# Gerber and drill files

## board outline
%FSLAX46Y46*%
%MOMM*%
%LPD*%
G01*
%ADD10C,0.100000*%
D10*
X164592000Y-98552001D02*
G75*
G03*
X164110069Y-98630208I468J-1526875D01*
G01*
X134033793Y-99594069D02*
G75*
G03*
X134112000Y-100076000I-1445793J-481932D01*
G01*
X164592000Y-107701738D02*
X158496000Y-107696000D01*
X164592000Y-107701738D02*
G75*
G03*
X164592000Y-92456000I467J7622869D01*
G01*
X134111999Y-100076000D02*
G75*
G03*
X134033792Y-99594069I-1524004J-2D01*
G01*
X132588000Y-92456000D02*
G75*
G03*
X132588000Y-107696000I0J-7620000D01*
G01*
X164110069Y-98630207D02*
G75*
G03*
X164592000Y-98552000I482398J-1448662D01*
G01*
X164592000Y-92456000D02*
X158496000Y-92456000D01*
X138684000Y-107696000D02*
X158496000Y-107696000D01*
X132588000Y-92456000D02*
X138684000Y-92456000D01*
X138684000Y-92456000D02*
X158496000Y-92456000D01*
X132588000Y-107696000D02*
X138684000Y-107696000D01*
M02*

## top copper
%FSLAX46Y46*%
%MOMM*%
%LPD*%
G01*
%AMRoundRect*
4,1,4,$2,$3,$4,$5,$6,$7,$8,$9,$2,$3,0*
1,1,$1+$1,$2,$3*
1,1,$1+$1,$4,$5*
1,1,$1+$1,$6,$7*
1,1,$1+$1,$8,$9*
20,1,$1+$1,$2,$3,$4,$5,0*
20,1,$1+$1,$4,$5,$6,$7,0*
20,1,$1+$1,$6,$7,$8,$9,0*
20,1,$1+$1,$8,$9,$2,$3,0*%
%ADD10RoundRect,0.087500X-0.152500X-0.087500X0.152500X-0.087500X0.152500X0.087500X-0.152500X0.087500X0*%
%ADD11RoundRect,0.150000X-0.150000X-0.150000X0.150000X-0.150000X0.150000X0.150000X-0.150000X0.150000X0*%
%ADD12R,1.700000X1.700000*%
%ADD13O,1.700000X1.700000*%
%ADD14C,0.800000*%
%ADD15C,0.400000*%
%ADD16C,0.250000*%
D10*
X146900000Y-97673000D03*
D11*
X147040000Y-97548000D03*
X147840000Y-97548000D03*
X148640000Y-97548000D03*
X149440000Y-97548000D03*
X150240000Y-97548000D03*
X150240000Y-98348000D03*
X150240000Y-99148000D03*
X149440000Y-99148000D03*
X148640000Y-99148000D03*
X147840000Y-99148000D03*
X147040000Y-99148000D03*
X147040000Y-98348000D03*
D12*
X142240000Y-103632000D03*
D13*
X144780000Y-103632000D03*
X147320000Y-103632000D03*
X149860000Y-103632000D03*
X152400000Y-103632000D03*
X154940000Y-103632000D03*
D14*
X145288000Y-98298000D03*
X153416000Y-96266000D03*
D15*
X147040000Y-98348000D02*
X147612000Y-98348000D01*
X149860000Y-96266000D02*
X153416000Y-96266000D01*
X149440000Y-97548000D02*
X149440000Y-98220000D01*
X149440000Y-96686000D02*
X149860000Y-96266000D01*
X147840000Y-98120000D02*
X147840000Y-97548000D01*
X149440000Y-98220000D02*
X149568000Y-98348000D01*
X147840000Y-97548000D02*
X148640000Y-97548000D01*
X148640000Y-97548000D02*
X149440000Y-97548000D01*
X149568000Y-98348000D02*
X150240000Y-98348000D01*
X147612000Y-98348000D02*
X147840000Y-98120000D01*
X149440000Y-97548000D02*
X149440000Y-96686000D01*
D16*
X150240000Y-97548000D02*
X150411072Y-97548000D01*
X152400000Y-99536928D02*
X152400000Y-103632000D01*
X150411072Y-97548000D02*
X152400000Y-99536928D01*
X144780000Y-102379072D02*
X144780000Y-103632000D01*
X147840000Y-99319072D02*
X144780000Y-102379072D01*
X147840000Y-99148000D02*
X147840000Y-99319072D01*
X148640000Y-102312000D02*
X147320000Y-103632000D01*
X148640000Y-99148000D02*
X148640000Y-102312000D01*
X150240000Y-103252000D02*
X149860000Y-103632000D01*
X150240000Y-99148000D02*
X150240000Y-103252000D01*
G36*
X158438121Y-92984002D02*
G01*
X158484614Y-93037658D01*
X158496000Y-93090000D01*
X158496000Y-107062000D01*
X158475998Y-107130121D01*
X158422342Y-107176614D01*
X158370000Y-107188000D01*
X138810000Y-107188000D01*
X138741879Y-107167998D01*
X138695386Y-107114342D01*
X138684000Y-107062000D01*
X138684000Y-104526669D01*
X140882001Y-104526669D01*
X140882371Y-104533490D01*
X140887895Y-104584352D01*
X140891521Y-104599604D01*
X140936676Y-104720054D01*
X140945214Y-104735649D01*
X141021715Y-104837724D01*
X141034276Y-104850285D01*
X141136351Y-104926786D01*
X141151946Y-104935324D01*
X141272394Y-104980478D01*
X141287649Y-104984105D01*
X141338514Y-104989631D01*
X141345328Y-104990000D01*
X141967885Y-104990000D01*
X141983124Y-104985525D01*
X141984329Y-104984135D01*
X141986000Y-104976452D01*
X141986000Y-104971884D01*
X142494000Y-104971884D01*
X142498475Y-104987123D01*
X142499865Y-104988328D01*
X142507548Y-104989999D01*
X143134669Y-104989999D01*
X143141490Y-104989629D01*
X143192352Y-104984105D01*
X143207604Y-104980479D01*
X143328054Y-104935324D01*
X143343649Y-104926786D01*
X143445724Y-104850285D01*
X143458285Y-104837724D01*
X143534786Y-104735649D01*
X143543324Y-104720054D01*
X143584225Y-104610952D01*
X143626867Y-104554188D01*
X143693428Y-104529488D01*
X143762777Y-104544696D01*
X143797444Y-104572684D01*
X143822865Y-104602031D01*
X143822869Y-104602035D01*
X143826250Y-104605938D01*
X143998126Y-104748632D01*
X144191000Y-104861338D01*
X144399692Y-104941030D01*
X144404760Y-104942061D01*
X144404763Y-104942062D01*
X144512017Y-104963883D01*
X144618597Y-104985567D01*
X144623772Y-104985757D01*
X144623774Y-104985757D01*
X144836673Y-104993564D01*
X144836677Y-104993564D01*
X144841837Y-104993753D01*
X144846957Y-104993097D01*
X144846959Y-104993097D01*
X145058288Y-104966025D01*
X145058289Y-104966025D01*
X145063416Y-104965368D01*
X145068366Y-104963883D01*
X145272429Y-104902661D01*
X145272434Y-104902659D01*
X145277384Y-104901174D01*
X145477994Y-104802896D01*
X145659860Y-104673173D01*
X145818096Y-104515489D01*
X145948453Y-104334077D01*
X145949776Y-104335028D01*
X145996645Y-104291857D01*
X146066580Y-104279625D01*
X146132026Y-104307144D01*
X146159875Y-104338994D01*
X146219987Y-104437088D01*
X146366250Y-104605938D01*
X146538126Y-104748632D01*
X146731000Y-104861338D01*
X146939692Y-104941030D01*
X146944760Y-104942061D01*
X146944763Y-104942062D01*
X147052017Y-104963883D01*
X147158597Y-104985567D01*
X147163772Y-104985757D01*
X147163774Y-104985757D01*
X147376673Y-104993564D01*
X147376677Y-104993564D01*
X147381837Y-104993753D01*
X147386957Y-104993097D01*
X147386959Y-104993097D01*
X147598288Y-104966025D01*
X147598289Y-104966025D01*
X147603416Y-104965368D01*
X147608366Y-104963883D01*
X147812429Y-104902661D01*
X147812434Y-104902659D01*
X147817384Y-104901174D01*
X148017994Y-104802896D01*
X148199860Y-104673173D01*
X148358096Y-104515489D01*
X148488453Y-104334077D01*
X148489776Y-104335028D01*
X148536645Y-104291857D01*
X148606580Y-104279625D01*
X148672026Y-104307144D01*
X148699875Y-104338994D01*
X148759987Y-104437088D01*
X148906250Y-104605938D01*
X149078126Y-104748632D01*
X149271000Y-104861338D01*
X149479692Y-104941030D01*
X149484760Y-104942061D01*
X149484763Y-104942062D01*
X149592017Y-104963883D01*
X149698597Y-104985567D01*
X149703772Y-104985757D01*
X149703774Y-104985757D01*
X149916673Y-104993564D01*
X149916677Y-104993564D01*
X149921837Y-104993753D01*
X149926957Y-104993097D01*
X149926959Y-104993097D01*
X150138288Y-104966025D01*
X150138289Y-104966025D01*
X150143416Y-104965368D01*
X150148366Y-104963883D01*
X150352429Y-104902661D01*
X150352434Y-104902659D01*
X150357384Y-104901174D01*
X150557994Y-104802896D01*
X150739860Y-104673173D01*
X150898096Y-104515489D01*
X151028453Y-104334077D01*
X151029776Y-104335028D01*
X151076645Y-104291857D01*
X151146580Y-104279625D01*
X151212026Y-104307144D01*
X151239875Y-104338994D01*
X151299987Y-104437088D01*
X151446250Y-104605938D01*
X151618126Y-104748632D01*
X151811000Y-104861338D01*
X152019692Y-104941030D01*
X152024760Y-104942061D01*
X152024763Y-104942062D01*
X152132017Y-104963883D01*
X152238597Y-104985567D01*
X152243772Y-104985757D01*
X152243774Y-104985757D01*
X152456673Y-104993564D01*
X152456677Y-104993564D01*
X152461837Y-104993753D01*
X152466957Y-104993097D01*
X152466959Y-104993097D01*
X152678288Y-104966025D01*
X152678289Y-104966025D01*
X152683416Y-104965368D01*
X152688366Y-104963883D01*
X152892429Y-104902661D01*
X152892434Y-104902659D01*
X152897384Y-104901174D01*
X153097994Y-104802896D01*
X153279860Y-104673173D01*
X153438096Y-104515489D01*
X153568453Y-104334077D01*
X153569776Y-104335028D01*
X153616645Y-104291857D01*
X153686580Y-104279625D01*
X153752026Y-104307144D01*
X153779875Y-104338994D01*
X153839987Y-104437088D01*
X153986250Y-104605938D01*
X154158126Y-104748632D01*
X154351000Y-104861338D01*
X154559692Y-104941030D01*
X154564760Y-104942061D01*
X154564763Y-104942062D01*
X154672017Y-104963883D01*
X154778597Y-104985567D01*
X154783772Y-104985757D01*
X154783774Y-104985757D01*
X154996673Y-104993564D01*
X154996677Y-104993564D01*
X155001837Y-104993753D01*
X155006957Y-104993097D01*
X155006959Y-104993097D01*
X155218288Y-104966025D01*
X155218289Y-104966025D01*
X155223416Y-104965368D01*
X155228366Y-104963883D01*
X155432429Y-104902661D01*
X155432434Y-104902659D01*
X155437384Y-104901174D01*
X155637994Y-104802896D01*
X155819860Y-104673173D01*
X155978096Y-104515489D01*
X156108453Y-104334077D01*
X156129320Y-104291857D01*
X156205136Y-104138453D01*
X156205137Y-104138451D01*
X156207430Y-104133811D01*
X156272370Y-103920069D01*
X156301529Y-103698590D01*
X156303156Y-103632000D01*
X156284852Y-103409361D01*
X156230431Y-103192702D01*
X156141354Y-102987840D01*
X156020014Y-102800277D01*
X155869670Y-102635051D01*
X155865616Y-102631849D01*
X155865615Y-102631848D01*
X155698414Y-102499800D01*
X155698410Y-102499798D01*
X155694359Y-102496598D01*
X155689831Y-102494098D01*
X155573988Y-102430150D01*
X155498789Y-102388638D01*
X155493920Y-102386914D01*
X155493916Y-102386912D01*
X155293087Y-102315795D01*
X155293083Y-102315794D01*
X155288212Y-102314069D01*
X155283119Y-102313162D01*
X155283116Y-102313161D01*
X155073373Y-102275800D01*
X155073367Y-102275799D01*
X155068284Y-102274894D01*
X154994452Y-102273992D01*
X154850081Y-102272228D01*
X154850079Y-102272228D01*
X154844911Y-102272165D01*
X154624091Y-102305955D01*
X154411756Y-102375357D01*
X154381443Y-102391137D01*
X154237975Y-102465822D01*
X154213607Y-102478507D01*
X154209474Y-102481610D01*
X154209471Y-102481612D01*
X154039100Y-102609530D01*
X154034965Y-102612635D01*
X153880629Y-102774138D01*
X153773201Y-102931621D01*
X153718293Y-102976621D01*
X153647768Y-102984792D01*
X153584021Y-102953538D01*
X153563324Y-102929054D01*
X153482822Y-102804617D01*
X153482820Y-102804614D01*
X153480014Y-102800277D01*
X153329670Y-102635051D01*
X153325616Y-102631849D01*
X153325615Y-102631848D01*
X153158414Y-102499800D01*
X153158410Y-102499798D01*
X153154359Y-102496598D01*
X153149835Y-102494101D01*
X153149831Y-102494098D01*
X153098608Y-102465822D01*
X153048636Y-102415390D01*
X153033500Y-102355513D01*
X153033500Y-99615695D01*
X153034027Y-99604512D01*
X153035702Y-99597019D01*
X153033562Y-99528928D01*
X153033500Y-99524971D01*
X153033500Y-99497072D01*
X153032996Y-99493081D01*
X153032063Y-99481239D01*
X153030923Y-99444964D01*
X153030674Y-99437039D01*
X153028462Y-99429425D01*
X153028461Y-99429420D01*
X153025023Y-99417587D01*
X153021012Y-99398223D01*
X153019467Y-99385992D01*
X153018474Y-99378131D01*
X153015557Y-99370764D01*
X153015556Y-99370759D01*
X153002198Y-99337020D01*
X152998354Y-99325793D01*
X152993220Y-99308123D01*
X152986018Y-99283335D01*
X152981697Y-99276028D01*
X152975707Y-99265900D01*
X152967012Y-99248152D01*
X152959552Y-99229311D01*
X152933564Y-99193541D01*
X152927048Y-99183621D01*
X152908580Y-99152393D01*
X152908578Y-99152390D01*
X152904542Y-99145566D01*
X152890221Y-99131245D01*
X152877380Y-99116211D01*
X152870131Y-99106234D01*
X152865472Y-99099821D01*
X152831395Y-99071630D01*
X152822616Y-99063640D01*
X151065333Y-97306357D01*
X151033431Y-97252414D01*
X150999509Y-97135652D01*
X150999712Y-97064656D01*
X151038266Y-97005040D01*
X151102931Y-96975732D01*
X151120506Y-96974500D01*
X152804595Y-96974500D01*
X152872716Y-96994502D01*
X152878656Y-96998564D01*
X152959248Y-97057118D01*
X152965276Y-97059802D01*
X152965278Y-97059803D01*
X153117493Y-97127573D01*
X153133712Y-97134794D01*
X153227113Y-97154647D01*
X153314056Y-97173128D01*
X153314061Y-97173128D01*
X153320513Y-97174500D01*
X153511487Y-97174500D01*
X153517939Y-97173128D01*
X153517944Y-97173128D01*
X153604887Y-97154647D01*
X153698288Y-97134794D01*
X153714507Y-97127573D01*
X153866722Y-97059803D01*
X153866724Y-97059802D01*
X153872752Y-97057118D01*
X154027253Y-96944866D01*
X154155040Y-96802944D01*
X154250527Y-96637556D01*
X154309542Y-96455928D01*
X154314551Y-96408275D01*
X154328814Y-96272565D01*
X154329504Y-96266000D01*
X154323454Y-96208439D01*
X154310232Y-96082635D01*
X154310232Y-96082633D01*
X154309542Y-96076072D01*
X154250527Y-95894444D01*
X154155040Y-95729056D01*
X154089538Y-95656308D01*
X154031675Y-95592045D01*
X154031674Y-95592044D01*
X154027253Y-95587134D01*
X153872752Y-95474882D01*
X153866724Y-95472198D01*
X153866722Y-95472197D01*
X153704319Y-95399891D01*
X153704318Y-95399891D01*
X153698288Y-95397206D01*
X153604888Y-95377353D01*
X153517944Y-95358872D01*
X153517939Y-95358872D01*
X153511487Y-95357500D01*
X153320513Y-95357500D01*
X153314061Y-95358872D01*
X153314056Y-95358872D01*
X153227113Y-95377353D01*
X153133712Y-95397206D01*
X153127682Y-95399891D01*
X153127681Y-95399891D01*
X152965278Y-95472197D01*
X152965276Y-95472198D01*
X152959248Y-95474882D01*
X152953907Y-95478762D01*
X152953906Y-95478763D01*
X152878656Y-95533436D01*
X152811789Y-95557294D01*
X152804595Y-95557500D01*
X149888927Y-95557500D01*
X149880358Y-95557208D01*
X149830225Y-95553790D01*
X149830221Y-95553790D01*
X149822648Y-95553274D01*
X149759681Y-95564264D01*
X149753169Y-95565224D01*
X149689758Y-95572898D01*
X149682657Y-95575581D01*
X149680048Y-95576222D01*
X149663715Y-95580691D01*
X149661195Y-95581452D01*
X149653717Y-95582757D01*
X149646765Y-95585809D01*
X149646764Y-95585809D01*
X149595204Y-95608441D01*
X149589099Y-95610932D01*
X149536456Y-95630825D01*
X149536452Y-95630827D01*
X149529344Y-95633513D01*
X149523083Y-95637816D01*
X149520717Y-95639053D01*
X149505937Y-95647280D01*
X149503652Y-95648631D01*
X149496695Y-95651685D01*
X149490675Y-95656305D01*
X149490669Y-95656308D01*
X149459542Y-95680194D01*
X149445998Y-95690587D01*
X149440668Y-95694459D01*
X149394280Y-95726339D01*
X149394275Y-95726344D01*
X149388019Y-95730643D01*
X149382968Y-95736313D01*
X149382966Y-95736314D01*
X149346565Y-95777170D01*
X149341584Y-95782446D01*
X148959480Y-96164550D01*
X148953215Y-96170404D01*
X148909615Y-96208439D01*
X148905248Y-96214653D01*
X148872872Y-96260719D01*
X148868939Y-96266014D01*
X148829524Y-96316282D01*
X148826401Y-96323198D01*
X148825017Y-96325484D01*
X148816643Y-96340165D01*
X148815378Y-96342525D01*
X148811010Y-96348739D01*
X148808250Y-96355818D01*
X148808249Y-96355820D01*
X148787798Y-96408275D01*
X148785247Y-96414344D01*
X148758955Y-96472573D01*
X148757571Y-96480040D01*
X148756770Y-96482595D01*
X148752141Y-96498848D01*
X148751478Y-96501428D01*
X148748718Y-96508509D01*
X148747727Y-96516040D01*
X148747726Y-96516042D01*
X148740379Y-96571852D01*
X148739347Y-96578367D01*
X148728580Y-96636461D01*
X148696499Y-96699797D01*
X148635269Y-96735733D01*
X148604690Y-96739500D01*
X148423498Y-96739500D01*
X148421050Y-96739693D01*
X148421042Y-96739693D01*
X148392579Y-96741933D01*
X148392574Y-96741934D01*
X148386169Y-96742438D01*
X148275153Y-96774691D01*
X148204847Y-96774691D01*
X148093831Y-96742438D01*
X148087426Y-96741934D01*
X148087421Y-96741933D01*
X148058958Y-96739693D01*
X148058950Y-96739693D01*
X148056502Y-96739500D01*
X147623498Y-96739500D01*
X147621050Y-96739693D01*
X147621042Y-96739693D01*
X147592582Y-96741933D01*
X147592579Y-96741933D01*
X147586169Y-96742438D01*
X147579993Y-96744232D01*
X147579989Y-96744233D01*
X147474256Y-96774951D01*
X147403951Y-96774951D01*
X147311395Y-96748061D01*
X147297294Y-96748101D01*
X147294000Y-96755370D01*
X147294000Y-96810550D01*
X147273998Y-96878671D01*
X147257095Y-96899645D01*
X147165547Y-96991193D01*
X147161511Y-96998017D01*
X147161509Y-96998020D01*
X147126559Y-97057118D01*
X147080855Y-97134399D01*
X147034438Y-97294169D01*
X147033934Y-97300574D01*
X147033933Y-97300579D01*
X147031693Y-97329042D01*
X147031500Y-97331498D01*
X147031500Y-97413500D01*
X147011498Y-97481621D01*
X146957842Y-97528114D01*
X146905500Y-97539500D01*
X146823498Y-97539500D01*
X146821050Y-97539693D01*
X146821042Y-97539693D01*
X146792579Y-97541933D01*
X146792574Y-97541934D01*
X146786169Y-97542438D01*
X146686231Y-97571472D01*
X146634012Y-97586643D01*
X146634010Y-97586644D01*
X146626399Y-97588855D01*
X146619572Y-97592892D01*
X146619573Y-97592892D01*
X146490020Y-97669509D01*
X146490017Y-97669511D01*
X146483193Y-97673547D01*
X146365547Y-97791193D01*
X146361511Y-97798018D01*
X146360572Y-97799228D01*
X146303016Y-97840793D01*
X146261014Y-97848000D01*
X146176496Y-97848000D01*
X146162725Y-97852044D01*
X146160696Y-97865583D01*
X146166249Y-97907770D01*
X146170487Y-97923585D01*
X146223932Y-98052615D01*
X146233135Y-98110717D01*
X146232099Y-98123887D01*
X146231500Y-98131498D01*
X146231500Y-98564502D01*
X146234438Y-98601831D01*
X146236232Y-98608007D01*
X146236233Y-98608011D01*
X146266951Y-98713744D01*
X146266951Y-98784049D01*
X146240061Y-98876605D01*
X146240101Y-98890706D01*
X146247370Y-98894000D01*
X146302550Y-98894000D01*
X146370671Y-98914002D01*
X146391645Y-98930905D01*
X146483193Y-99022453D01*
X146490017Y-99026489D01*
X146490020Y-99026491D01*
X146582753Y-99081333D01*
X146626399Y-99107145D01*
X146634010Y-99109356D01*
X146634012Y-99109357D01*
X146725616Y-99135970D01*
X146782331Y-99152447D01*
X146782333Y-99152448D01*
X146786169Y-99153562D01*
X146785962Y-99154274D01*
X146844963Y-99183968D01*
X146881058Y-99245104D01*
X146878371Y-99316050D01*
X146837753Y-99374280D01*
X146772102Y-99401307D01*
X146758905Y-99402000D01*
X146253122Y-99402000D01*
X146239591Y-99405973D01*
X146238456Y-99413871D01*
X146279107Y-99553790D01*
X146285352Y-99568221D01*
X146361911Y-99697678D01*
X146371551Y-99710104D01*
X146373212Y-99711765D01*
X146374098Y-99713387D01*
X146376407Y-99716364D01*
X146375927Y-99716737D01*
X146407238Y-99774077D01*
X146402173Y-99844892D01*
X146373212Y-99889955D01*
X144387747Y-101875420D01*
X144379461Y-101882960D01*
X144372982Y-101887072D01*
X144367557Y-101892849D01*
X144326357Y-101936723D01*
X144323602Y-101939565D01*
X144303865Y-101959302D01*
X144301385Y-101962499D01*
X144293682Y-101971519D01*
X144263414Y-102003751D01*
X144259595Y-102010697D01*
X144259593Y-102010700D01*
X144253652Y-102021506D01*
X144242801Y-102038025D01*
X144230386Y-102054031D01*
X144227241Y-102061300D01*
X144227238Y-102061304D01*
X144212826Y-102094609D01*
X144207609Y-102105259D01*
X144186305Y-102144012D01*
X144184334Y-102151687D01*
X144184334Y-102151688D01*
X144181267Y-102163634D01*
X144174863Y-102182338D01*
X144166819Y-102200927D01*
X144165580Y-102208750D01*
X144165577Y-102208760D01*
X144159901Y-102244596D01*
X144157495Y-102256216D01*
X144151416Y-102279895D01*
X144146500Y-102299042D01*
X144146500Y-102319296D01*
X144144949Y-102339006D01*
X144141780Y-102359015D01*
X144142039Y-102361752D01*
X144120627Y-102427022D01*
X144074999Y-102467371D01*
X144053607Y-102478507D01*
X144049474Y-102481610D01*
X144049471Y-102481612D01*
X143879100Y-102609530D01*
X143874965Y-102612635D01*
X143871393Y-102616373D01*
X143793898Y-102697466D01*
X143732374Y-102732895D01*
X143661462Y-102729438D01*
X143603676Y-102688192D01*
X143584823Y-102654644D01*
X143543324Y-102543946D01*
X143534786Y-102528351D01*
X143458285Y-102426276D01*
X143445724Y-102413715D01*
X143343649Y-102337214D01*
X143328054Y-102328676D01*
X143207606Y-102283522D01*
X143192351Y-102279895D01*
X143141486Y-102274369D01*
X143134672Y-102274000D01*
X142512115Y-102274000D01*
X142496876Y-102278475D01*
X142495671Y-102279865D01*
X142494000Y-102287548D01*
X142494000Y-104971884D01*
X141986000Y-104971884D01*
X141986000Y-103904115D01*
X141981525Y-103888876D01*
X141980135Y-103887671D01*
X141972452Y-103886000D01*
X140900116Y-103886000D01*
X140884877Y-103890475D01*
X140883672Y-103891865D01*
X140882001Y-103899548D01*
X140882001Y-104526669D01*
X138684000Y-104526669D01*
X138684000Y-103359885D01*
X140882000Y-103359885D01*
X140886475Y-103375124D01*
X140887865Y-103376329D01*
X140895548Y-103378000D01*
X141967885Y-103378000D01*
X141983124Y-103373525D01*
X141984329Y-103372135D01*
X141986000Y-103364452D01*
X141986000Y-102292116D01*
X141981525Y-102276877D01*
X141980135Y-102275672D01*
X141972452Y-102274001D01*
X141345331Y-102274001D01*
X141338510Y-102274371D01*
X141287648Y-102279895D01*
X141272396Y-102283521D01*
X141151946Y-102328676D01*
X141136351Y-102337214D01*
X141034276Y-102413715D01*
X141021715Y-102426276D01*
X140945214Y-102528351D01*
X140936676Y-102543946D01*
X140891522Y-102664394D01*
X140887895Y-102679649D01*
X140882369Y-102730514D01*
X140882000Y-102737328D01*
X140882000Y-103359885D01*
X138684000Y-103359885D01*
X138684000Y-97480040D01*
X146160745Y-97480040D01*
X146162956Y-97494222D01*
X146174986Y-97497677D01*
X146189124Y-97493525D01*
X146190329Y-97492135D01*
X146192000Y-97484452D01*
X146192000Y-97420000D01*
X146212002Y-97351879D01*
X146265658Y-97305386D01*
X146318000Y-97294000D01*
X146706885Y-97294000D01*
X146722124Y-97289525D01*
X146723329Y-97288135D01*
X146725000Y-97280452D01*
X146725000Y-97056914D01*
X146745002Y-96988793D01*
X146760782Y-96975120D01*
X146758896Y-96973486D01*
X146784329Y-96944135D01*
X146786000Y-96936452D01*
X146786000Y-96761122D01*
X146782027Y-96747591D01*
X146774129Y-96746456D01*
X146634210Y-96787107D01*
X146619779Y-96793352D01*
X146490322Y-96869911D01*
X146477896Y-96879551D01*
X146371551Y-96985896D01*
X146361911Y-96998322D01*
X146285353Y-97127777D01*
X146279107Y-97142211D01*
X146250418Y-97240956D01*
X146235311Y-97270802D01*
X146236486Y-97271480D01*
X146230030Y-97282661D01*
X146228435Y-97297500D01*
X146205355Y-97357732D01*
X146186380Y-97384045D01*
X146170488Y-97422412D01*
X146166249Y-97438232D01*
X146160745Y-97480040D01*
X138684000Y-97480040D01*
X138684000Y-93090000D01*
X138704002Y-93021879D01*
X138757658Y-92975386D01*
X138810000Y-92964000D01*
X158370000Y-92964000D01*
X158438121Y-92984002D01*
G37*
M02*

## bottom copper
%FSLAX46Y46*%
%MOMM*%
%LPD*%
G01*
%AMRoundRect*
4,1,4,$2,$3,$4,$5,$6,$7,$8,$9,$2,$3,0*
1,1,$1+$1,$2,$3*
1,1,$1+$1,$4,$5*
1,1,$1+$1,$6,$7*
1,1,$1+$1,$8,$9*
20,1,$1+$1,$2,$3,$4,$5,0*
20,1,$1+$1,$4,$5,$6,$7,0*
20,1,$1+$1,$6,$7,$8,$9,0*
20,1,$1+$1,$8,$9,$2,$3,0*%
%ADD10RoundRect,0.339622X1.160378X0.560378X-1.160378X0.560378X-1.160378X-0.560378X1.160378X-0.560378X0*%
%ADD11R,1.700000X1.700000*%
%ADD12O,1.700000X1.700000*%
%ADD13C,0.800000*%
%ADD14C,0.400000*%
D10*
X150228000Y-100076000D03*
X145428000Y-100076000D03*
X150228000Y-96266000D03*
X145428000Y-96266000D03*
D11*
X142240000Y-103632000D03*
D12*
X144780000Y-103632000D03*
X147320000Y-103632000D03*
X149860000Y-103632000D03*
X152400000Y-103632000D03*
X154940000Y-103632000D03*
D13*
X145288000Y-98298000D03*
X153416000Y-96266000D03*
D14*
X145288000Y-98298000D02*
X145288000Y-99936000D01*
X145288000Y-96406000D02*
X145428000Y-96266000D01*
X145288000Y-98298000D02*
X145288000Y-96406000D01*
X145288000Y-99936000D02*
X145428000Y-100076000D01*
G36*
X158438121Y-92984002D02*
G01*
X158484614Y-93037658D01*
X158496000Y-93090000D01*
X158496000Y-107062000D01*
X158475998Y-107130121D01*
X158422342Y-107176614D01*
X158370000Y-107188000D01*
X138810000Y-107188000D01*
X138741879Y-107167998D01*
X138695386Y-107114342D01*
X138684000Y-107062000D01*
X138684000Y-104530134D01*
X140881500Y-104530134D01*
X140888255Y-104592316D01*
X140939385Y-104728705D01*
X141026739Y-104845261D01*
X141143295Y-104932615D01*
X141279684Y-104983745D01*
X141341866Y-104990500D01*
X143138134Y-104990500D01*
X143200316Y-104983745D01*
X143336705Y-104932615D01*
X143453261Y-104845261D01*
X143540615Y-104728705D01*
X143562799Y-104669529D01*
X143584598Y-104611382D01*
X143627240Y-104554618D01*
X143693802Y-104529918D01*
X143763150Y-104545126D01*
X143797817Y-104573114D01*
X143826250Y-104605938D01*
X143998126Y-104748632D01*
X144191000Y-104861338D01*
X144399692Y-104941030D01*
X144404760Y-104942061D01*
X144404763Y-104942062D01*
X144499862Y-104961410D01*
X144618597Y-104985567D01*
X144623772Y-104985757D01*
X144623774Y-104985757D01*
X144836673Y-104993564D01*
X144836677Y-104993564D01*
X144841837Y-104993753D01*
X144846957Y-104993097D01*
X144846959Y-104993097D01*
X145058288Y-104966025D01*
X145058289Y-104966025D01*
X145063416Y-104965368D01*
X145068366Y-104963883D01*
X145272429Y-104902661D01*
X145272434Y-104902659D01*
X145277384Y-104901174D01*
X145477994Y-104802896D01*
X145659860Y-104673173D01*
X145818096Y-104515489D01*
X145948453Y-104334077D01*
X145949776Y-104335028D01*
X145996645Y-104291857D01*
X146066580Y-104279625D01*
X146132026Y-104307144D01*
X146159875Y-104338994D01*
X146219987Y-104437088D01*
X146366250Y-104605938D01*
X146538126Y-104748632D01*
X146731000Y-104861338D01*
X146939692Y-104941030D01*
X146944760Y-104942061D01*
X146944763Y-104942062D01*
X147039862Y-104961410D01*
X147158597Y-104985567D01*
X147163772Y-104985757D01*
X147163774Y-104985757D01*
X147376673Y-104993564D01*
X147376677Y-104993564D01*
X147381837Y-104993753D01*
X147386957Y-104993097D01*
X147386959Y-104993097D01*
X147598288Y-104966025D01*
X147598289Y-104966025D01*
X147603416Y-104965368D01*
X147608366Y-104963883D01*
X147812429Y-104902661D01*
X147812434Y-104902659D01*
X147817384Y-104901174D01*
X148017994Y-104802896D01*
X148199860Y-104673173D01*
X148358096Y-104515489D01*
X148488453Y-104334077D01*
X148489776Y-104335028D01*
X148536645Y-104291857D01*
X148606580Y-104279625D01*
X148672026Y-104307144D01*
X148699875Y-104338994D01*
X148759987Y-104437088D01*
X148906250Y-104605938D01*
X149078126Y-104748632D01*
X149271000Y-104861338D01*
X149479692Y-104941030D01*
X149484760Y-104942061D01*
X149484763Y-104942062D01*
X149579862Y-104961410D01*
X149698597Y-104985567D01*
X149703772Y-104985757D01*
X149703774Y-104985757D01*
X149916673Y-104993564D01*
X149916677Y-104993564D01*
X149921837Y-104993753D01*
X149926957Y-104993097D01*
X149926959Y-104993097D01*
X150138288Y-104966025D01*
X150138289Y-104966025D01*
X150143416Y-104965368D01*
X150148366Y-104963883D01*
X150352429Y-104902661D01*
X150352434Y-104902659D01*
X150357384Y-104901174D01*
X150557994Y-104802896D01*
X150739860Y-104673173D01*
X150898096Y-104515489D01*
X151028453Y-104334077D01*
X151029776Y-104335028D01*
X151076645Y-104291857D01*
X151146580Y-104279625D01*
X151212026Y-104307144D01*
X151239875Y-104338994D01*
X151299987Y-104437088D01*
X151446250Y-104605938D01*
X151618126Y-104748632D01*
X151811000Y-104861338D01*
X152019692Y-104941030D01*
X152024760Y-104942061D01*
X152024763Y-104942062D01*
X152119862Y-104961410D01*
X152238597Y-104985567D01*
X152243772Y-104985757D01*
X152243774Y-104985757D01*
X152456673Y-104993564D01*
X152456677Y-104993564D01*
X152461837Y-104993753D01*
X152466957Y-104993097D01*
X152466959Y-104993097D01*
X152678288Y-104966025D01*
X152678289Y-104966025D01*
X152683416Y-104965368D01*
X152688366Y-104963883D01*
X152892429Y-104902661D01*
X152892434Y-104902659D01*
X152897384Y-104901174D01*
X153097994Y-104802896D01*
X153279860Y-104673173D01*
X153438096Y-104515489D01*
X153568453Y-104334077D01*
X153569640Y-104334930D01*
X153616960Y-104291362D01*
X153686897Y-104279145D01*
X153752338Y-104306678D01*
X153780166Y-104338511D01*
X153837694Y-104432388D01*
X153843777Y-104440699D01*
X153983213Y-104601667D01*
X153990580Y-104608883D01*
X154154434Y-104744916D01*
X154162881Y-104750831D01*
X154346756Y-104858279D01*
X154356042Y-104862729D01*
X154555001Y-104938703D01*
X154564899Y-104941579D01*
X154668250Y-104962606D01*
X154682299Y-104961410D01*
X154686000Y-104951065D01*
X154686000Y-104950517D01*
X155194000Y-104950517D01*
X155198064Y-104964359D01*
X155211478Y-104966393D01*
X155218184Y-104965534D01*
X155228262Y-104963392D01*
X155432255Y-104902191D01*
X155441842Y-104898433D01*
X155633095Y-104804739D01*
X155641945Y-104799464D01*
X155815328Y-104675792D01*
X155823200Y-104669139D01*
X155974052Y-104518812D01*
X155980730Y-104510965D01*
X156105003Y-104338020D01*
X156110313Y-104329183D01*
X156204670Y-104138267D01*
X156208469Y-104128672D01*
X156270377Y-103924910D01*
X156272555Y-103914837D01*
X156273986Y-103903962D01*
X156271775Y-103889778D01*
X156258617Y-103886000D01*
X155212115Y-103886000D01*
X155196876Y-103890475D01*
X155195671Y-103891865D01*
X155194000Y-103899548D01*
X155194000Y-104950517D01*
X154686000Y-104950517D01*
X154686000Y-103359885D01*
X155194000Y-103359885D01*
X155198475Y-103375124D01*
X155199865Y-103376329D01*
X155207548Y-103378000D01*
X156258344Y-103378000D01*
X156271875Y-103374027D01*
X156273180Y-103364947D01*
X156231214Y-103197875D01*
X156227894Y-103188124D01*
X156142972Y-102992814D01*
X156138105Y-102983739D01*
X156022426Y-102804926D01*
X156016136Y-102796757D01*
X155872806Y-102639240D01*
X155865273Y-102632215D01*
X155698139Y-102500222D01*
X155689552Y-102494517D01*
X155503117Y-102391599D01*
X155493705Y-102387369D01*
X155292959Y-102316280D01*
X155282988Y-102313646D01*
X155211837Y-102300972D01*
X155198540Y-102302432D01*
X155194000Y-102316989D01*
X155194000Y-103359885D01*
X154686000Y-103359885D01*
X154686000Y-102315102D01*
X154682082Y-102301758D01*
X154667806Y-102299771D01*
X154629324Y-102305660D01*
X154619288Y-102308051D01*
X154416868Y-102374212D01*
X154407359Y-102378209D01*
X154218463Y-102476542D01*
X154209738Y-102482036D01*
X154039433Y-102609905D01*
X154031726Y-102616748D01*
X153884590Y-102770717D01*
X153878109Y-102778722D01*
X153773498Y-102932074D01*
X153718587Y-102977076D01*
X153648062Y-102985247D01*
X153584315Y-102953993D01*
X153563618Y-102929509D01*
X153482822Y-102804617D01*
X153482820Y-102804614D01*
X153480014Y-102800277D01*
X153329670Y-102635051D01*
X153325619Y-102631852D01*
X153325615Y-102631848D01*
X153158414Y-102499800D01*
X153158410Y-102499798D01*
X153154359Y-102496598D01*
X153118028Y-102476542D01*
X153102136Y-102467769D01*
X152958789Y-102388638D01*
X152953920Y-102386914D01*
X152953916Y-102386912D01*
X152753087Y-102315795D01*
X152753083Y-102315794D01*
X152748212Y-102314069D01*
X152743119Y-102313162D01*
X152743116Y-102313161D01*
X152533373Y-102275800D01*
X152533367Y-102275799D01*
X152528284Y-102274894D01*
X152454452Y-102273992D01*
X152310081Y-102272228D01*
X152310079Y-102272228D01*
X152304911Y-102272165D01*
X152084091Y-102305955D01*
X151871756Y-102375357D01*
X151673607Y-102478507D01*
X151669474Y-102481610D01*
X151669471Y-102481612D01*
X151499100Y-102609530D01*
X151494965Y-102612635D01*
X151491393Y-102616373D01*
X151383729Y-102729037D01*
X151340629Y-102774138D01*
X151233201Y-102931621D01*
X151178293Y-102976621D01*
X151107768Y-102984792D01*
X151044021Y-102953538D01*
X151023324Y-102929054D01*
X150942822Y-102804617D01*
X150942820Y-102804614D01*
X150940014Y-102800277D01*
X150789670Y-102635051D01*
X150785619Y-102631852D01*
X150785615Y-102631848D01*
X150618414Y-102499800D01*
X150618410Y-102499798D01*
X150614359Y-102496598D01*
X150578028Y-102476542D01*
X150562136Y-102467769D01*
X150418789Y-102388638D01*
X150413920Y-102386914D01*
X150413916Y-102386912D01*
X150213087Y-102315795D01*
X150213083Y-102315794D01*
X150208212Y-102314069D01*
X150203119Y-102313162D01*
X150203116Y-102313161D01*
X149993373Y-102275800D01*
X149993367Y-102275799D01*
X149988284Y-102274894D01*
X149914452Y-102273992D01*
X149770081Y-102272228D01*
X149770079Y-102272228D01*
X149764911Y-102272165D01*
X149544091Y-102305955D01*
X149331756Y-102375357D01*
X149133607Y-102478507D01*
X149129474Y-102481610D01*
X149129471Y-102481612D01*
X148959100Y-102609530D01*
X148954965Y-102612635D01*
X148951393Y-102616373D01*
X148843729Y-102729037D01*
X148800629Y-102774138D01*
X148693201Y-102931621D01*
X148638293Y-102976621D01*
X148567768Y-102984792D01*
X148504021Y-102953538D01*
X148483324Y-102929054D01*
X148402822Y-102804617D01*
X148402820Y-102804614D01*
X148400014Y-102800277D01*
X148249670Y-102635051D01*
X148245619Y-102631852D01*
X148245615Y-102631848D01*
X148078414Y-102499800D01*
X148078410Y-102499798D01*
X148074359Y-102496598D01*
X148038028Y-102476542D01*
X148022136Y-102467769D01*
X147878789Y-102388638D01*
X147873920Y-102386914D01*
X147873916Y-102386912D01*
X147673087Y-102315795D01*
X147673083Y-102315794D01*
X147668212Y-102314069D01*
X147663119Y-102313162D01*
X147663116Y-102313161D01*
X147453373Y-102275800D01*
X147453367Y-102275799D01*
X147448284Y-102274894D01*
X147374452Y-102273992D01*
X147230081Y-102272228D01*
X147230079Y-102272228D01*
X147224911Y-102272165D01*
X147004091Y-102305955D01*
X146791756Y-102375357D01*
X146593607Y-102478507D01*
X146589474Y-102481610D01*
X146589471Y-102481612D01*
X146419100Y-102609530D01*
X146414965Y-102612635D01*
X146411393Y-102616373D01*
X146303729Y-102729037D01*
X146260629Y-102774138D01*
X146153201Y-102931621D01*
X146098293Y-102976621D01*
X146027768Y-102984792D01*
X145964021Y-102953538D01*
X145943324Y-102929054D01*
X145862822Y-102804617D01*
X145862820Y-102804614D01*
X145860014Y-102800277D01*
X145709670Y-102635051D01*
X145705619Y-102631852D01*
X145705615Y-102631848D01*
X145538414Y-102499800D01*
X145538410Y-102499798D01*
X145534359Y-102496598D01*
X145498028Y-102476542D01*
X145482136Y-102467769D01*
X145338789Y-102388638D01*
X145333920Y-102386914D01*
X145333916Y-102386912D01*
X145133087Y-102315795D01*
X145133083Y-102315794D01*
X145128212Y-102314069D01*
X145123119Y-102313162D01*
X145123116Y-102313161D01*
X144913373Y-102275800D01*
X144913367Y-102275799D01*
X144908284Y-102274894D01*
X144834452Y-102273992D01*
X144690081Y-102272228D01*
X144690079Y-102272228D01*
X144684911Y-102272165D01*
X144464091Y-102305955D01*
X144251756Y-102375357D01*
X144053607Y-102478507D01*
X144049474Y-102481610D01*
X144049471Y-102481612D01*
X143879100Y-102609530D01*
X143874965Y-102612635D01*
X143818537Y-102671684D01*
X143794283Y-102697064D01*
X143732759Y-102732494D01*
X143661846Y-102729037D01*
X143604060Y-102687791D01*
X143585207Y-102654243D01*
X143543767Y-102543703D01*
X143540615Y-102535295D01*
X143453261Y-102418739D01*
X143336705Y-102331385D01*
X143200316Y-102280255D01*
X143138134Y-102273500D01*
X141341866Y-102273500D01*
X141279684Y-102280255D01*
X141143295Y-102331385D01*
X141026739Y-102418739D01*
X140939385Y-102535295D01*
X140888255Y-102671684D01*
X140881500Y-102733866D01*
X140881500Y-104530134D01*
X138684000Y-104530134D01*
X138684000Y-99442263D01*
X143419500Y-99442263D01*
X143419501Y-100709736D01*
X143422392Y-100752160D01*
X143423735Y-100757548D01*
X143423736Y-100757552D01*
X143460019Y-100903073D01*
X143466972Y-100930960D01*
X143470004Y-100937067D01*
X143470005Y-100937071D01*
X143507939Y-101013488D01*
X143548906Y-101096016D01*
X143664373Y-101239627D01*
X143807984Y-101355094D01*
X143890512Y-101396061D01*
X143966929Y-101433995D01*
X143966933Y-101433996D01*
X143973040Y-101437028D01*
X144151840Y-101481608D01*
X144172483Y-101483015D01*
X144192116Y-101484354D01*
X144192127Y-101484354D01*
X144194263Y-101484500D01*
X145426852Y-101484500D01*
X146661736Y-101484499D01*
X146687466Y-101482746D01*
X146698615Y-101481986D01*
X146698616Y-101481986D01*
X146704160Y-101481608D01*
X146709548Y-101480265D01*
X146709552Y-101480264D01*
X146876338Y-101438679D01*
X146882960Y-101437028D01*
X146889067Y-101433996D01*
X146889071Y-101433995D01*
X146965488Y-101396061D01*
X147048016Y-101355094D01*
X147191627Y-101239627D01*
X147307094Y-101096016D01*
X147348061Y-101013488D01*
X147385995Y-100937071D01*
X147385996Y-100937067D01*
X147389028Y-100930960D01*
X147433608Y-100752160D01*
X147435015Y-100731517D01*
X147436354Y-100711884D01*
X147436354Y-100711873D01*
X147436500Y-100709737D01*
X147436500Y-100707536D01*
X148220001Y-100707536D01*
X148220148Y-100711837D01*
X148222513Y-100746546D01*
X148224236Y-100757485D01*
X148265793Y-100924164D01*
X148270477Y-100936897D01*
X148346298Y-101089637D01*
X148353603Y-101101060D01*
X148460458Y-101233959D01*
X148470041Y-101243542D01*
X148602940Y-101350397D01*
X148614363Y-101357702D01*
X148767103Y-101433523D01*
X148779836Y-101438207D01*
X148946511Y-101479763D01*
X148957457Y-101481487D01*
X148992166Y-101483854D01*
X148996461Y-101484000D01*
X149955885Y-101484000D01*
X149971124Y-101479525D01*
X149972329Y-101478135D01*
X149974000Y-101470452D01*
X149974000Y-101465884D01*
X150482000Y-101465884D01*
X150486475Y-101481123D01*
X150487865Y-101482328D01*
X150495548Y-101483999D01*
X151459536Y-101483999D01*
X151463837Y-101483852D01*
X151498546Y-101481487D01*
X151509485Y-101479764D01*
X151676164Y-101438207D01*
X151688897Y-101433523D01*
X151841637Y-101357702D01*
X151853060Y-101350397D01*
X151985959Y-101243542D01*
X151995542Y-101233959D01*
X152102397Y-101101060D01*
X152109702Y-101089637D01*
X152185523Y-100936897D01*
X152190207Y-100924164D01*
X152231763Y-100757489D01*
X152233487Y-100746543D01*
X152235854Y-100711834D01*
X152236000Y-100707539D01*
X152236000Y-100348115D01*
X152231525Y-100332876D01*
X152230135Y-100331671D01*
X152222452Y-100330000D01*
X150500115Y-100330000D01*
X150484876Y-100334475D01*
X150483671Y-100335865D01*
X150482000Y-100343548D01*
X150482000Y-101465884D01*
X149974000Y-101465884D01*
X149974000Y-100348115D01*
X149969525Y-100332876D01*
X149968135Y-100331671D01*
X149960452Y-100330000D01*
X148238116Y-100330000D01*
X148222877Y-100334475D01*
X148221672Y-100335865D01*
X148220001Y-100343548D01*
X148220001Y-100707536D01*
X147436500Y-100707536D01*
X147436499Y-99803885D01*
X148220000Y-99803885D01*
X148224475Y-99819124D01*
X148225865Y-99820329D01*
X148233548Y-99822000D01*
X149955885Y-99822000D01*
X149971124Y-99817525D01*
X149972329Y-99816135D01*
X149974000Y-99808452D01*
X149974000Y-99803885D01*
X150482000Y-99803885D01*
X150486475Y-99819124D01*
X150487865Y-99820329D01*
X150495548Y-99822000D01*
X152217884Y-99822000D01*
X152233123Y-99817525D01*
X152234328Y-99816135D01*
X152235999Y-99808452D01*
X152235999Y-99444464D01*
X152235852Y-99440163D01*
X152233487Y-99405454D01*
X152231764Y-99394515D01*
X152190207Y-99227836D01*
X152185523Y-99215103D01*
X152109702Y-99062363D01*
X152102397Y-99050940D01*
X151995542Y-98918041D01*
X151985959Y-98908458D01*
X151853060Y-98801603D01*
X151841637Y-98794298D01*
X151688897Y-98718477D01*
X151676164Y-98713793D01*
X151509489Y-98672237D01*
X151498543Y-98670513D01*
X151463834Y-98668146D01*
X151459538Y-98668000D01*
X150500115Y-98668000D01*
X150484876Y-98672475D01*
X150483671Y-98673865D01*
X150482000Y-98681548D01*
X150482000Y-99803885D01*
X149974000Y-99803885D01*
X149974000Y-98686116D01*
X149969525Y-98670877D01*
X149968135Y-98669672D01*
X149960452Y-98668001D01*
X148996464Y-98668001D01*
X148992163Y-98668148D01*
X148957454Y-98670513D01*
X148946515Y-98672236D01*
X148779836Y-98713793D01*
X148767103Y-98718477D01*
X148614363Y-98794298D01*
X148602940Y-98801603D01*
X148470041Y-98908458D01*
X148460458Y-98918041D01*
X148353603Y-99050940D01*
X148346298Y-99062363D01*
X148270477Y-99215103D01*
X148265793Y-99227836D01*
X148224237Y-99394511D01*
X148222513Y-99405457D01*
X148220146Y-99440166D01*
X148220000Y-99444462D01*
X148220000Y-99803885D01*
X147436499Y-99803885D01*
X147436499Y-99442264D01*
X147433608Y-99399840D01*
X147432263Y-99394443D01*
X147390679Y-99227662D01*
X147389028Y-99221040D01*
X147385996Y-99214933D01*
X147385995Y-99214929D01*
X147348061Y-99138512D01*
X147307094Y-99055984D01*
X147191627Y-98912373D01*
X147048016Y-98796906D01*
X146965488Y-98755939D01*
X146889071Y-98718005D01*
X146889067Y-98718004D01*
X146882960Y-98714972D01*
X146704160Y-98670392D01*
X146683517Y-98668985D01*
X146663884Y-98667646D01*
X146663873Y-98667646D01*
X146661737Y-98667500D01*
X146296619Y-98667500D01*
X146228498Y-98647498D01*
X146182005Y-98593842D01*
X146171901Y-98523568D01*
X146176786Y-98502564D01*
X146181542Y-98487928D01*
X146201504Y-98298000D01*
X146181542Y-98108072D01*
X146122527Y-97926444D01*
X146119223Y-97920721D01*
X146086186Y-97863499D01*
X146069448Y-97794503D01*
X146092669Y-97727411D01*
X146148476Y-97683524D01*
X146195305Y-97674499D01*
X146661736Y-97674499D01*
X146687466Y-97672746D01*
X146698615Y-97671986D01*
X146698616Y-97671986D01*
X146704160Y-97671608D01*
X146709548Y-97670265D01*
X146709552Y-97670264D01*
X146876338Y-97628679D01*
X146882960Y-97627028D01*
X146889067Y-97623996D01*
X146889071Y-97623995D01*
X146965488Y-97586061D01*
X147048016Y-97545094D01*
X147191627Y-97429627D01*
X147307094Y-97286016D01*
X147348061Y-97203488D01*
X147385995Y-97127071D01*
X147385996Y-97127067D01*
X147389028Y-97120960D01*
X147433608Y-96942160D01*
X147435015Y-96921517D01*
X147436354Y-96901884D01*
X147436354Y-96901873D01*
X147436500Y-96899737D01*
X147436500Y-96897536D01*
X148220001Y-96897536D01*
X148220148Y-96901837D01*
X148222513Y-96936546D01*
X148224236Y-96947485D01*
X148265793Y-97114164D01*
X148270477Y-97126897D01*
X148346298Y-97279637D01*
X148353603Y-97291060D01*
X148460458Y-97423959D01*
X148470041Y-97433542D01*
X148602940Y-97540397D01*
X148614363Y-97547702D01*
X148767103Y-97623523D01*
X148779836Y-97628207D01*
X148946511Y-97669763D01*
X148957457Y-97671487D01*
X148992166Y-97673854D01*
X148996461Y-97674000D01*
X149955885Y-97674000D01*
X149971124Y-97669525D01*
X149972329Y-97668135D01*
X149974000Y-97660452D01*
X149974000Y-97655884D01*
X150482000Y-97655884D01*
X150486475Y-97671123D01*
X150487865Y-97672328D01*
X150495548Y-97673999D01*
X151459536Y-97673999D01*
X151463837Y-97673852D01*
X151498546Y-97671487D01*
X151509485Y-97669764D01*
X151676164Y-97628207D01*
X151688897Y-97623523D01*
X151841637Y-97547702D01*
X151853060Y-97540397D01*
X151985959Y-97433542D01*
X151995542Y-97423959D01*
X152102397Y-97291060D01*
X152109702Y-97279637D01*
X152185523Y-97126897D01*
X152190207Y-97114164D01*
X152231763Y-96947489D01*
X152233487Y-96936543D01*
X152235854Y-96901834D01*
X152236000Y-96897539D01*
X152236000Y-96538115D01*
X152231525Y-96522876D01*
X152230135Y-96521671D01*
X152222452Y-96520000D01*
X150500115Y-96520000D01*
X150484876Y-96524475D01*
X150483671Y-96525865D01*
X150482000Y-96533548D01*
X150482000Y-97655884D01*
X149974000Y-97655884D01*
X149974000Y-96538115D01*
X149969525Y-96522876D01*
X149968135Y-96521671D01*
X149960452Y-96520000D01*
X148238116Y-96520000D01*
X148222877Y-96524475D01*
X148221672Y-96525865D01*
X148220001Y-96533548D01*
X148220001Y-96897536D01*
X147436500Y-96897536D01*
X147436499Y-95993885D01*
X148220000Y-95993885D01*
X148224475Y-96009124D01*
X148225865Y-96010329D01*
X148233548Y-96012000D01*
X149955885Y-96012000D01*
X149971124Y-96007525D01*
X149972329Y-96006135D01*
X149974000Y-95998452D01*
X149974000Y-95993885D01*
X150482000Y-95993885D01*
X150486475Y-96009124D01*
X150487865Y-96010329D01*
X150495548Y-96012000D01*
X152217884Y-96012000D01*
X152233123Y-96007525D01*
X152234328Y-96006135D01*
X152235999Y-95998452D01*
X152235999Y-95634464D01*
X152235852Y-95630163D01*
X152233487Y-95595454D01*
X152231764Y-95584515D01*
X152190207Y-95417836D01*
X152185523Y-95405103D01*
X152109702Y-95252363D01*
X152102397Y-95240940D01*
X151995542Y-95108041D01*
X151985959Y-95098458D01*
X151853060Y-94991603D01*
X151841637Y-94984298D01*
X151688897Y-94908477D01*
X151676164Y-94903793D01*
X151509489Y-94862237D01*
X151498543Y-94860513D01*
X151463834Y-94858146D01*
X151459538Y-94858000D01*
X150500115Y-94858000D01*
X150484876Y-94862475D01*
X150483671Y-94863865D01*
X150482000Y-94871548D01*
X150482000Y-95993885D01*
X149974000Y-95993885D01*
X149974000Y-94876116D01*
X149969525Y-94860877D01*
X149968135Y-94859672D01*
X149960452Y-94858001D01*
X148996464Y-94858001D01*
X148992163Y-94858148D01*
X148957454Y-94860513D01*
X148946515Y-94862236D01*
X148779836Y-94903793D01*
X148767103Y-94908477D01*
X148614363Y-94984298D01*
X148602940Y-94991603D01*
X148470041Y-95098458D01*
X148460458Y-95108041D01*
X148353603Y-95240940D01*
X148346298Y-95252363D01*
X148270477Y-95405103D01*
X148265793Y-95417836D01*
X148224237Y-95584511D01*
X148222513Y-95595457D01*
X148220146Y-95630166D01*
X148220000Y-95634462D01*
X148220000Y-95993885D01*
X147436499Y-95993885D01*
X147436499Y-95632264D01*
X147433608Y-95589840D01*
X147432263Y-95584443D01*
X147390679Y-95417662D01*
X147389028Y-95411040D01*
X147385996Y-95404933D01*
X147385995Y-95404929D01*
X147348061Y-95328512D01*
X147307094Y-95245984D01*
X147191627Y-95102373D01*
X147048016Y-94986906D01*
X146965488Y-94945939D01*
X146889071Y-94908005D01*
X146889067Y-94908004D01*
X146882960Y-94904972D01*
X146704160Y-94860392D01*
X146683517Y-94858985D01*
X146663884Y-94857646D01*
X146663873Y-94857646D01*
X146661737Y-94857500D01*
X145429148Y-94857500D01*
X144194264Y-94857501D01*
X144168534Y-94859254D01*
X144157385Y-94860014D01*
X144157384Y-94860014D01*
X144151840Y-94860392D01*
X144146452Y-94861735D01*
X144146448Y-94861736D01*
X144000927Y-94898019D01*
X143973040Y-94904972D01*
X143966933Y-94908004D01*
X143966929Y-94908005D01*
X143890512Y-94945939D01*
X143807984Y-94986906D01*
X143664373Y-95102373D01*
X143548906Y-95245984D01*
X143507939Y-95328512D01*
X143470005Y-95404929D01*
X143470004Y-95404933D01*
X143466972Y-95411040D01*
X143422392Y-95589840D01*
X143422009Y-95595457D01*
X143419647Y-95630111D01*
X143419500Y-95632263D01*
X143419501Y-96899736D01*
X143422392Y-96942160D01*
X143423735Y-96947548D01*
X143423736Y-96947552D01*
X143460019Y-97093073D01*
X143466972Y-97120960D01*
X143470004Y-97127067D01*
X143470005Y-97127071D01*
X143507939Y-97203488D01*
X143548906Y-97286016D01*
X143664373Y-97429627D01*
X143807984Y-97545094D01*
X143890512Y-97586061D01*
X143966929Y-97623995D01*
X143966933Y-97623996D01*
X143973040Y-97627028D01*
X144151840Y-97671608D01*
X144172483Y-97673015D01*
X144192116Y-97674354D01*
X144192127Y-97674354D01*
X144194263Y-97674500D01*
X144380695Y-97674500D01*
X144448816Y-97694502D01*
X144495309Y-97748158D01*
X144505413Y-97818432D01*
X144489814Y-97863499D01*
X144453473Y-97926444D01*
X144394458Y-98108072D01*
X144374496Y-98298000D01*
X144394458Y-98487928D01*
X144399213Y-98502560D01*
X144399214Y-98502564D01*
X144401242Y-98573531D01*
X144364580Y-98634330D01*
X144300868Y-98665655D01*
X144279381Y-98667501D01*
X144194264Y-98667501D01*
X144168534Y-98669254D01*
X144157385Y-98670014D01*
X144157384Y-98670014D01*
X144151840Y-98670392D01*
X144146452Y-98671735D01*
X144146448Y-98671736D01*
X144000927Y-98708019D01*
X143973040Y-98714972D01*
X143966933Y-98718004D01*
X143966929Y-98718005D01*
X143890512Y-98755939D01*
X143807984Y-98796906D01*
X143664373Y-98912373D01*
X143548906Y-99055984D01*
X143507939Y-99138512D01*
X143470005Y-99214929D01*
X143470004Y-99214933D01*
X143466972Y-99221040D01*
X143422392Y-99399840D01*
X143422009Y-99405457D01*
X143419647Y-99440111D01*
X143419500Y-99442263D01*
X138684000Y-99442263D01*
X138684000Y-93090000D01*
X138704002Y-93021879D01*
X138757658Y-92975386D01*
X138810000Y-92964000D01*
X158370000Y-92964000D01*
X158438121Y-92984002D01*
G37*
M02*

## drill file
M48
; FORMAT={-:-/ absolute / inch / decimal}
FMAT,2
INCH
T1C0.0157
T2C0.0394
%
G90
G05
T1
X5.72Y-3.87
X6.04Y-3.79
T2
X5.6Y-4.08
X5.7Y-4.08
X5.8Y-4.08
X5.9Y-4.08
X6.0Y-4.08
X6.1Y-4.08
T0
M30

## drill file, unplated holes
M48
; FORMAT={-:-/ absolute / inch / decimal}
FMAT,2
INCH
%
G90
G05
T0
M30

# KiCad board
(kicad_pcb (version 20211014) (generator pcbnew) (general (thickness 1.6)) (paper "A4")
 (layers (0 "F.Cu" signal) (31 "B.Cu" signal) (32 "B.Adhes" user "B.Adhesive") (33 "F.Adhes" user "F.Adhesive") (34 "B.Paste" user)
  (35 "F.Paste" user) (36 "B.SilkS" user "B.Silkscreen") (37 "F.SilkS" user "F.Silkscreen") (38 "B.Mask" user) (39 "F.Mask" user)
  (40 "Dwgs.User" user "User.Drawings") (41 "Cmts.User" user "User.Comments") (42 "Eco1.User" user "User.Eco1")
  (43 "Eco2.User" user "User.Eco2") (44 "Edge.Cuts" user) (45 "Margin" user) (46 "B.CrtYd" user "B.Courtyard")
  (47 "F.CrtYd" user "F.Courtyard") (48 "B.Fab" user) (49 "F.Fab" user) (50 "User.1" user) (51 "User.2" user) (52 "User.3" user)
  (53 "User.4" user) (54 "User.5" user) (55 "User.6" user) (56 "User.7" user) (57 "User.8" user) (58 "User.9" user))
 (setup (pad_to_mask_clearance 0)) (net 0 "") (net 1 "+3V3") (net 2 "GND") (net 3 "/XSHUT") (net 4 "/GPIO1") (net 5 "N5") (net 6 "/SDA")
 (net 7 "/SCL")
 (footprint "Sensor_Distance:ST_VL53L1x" (layer "F.Cu") (at 148.59 98.298)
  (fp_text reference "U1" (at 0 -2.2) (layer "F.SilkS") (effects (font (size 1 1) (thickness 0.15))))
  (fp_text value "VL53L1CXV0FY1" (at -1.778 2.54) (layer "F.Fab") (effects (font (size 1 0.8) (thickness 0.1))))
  (pad "1" smd roundrect (at -1.69 -0.625) (size 0.48 0.35) (layers "F.Cu" "F.Paste" "F.Mask") (roundrect_rratio 0.25) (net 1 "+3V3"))
  (pad "1" smd roundrect (at -1.55 -0.75) (size 0.6 0.6) (layers "F.Cu" "F.Paste" "F.Mask") (roundrect_rratio 0.25) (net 1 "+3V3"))
  (pad "2" smd roundrect (at -0.75 -0.75) (size 0.6 0.6) (layers "F.Cu" "F.Paste" "F.Mask") (roundrect_rratio 0.25) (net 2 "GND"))
  (pad "3" smd roundrect (at 0.05 -0.75) (size 0.6 0.6) (layers "F.Cu" "F.Paste" "F.Mask") (roundrect_rratio 0.25) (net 2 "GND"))
  (pad "4" smd roundrect (at 0.85 -0.75) (size 0.6 0.6) (layers "F.Cu" "F.Paste" "F.Mask") (roundrect_rratio 0.25) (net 2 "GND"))
  (pad "5" smd roundrect (at 1.65 -0.75) (size 0.6 0.6) (layers "F.Cu" "F.Paste" "F.Mask") (roundrect_rratio 0.25) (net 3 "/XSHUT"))
  (pad "6" smd roundrect (at 1.65 0.05) (size 0.6 0.6) (layers "F.Cu" "F.Paste" "F.Mask") (roundrect_rratio 0.25) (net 2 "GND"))
  (pad "7" smd roundrect (at 1.65 0.85) (size 0.6 0.6) (layers "F.Cu" "F.Paste" "F.Mask") (roundrect_rratio 0.25) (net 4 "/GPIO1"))
  (pad "8" smd roundrect (at 0.85 0.85) (size 0.6 0.6) (layers "F.Cu" "F.Paste" "F.Mask") (roundrect_rratio 0.25) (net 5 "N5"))
  (pad "9" smd roundrect (at 0.05 0.85) (size 0.6 0.6) (layers "F.Cu" "F.Paste" "F.Mask") (roundrect_rratio 0.25) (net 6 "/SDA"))
  (pad "10" smd roundrect (at -0.75 0.85) (size 0.6 0.6) (layers "F.Cu" "F.Paste" "F.Mask") (roundrect_rratio 0.25) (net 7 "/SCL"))
  (pad "11" smd roundrect (at -1.55 0.85) (size 0.6 0.6) (layers "F.Cu" "F.Paste" "F.Mask") (roundrect_rratio 0.25) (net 1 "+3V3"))
  (pad "12" smd roundrect (at -1.55 0.05) (size 0.6 0.6) (layers "F.Cu" "F.Paste" "F.Mask") (roundrect_rratio 0.25) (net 2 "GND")))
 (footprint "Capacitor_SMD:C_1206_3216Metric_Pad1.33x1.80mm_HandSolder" (layer "B.Cu") (at 147.828 100.076 180)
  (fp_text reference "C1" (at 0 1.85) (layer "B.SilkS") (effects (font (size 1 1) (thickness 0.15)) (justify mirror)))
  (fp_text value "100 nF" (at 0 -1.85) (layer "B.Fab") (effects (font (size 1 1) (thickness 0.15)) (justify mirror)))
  (pad "1" smd roundrect (at -2.4 0 180) (size 3 1.8) (layers "B.Cu" "B.Paste" "B.Mask") (roundrect_rratio 0.1886788889) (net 2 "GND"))
  (pad "2" smd roundrect (at 2.4 0 180) (size 3 1.8) (layers "B.Cu" "B.Paste" "B.Mask") (roundrect_rratio 0.1886788889) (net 1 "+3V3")))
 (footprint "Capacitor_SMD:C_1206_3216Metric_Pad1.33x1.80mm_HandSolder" (layer "B.Cu") (at 147.828 96.266 180)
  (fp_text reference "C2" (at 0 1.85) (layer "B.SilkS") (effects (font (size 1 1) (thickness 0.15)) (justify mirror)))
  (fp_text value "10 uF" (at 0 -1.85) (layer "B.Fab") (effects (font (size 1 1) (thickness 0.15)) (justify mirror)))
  (pad "1" smd roundrect (at -2.4 0 180) (size 3 1.8) (layers "B.Cu" "B.Paste" "B.Mask") (roundrect_rratio 0.1886788889) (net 2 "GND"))
  (pad "2" smd roundrect (at 2.4 0 180) (size 3 1.8) (layers "B.Cu" "B.Paste" "B.Mask") (roundrect_rratio 0.1886788889) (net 1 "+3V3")))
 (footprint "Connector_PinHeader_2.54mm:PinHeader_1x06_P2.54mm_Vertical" (layer "B.Cu") (at 142.24 103.632 -90)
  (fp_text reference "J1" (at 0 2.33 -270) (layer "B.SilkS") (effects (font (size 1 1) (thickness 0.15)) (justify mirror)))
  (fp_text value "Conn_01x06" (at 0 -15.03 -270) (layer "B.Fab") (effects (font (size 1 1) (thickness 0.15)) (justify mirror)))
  (pad "1" thru_hole rect (at 0 0 270) (size 1.7 1.7) (drill 1) (layers *.Cu *.Mask) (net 1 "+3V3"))
  (pad "2" thru_hole oval (at 0 -2.54 270) (size 1.7 1.7) (drill 1) (layers *.Cu *.Mask) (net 7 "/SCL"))
  (pad "3" thru_hole oval (at 0 -5.08 270) (size 1.7 1.7) (drill 1) (layers *.Cu *.Mask) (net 6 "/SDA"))
  (pad "4" thru_hole oval (at 0 -7.62 270) (size 1.7 1.7) (drill 1) (layers *.Cu *.Mask) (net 4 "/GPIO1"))
  (pad "5" thru_hole oval (at 0 -10.16 270) (size 1.7 1.7) (drill 1) (layers *.Cu *.Mask) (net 3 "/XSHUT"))
  (pad "6" thru_hole oval (at 0 -12.7 270) (size 1.7 1.7) (drill 1) (layers *.Cu *.Mask) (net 2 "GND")))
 (gr_arc (start 164.110069 98.630208) (mid 164.347888 98.571717) (end 164.592 98.552001) (layer "Edge.Cuts") (width 0.1))
 (gr_arc (start 134.112 100.076) (mid 131.083679 100.32012) (end 134.033793 99.594069) (layer "Edge.Cuts") (width 0.1))
 (gr_line (start 164.592 107.701738) (end 158.496 107.696) (layer "Edge.Cuts") (width 0.1))
 (gr_arc (start 164.592 92.456) (mid 172.215336 100.078869) (end 164.592 107.701738) (layer "Edge.Cuts") (width 0.1))
 (gr_arc (start 134.033792 99.594069) (mid 134.09232 99.831882) (end 134.111999 100.076) (layer "Edge.Cuts") (width 0.1))
 (gr_arc (start 132.588 107.696) (mid 124.968 100.076) (end 132.588 92.456) (layer "Edge.Cuts") (width 0.1))
 (gr_arc (start 164.592 98.552) (mid 164.837046 101.586022) (end 164.110069 98.630207) (layer "Edge.Cuts") (width 0.1))
 (gr_line (start 164.592 92.456) (end 158.496 92.456) (layer "Edge.Cuts") (width 0.1))
 (gr_line (start 138.684 107.696) (end 158.496 107.696) (layer "Edge.Cuts") (width 0.1))
 (gr_line (start 132.588 92.456) (end 138.684 92.456) (layer "Edge.Cuts") (width 0.1))
 (gr_line (start 138.684 92.456) (end 158.496 92.456) (layer "Edge.Cuts") (width 0.1))
 (gr_line (start 132.588 107.696) (end 138.684 107.696) (layer "Edge.Cuts") (width 0.1))
 (via (at 145.288 98.298) (size 0.8) (drill 0.4) (layers "F.Cu" "B.Cu") (free) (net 1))
 (segment (start 145.288 98.298) (end 145.288 99.936) (width 0.4) (layer "B.Cu") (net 1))
 (segment (start 145.288 96.406) (end 145.428 96.266) (width 0.4) (layer "B.Cu") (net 1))
 (segment (start 145.288 98.298) (end 145.288 96.406) (width 0.4) (layer "B.Cu") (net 1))
 (segment (start 145.288 99.936) (end 145.428 100.076) (width 0.4) (layer "B.Cu") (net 1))
 (segment (start 147.04 98.348) (end 147.612 98.348) (width 0.4) (layer "F.Cu") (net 2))
 (segment (start 149.86 96.266) (end 153.416 96.266) (width 0.4) (layer "F.Cu") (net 2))
 (segment (start 149.44 97.548) (end 149.44 98.22) (width 0.4) (layer "F.Cu") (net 2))
 (segment (start 149.44 96.686) (end 149.86 96.266) (width 0.4) (layer "F.Cu") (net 2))
 (segment (start 147.84 98.12) (end 147.84 97.548) (width 0.4) (layer "F.Cu") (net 2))
 (segment (start 149.44 98.22) (end 149.568 98.348) (width 0.4) (layer "F.Cu") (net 2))
 (segment (start 147.84 97.548) (end 148.64 97.548) (width 0.4) (layer "F.Cu") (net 2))
 (segment (start 148.64 97.548) (end 149.44 97.548) (width 0.4) (layer "F.Cu") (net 2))
 (segment (start 149.568 98.348) (end 150.24 98.348) (width 0.4) (layer "F.Cu") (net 2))
 (segment (start 147.612 98.348) (end 147.84 98.12) (width 0.4) (layer "F.Cu") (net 2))
 (segment (start 149.44 97.548) (end 149.44 96.686) (width 0.4) (layer "F.Cu") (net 2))
 (via (at 153.416 96.266) (size 0.8) (drill 0.4) (layers "F.Cu" "B.Cu") (free) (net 2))
 (segment (start 150.24 97.548) (end 150.411072 97.548) (width 0.25) (layer "F.Cu") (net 3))
 (segment (start 152.4 99.536928) (end 152.4 103.632) (width 0.25) (layer "F.Cu") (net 3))
 (segment (start 150.411072 97.548) (end 152.4 99.536928) (width 0.25) (layer "F.Cu") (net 3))
 (segment (start 144.78 102.379072) (end 144.78 103.632) (width 0.25) (layer "F.Cu") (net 7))
 (segment (start 147.84 99.319072) (end 144.78 102.379072) (width 0.25) (layer "F.Cu") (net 7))
 (segment (start 147.84 99.148) (end 147.84 99.319072) (width 0.25) (layer "F.Cu") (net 7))
 (segment (start 148.64 102.312) (end 147.32 103.632) (width 0.25) (layer "F.Cu") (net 6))
 (segment (start 148.64 99.148) (end 148.64 102.312) (width 0.25) (layer "F.Cu") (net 6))
 (segment (start 150.24 103.252) (end 149.86 103.632) (width 0.25) (layer "F.Cu") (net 4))
 (segment (start 150.24 99.148) (end 150.24 103.252) (width 0.25) (layer "F.Cu") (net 4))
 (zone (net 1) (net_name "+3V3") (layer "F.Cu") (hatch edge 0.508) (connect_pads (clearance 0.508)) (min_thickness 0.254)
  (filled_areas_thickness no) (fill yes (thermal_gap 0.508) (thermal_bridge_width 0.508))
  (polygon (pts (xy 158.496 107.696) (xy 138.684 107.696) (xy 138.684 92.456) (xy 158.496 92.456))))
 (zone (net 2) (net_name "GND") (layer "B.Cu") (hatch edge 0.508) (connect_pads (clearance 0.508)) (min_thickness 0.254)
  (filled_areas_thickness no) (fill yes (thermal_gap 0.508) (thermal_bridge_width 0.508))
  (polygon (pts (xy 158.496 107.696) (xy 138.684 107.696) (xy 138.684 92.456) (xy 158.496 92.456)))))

